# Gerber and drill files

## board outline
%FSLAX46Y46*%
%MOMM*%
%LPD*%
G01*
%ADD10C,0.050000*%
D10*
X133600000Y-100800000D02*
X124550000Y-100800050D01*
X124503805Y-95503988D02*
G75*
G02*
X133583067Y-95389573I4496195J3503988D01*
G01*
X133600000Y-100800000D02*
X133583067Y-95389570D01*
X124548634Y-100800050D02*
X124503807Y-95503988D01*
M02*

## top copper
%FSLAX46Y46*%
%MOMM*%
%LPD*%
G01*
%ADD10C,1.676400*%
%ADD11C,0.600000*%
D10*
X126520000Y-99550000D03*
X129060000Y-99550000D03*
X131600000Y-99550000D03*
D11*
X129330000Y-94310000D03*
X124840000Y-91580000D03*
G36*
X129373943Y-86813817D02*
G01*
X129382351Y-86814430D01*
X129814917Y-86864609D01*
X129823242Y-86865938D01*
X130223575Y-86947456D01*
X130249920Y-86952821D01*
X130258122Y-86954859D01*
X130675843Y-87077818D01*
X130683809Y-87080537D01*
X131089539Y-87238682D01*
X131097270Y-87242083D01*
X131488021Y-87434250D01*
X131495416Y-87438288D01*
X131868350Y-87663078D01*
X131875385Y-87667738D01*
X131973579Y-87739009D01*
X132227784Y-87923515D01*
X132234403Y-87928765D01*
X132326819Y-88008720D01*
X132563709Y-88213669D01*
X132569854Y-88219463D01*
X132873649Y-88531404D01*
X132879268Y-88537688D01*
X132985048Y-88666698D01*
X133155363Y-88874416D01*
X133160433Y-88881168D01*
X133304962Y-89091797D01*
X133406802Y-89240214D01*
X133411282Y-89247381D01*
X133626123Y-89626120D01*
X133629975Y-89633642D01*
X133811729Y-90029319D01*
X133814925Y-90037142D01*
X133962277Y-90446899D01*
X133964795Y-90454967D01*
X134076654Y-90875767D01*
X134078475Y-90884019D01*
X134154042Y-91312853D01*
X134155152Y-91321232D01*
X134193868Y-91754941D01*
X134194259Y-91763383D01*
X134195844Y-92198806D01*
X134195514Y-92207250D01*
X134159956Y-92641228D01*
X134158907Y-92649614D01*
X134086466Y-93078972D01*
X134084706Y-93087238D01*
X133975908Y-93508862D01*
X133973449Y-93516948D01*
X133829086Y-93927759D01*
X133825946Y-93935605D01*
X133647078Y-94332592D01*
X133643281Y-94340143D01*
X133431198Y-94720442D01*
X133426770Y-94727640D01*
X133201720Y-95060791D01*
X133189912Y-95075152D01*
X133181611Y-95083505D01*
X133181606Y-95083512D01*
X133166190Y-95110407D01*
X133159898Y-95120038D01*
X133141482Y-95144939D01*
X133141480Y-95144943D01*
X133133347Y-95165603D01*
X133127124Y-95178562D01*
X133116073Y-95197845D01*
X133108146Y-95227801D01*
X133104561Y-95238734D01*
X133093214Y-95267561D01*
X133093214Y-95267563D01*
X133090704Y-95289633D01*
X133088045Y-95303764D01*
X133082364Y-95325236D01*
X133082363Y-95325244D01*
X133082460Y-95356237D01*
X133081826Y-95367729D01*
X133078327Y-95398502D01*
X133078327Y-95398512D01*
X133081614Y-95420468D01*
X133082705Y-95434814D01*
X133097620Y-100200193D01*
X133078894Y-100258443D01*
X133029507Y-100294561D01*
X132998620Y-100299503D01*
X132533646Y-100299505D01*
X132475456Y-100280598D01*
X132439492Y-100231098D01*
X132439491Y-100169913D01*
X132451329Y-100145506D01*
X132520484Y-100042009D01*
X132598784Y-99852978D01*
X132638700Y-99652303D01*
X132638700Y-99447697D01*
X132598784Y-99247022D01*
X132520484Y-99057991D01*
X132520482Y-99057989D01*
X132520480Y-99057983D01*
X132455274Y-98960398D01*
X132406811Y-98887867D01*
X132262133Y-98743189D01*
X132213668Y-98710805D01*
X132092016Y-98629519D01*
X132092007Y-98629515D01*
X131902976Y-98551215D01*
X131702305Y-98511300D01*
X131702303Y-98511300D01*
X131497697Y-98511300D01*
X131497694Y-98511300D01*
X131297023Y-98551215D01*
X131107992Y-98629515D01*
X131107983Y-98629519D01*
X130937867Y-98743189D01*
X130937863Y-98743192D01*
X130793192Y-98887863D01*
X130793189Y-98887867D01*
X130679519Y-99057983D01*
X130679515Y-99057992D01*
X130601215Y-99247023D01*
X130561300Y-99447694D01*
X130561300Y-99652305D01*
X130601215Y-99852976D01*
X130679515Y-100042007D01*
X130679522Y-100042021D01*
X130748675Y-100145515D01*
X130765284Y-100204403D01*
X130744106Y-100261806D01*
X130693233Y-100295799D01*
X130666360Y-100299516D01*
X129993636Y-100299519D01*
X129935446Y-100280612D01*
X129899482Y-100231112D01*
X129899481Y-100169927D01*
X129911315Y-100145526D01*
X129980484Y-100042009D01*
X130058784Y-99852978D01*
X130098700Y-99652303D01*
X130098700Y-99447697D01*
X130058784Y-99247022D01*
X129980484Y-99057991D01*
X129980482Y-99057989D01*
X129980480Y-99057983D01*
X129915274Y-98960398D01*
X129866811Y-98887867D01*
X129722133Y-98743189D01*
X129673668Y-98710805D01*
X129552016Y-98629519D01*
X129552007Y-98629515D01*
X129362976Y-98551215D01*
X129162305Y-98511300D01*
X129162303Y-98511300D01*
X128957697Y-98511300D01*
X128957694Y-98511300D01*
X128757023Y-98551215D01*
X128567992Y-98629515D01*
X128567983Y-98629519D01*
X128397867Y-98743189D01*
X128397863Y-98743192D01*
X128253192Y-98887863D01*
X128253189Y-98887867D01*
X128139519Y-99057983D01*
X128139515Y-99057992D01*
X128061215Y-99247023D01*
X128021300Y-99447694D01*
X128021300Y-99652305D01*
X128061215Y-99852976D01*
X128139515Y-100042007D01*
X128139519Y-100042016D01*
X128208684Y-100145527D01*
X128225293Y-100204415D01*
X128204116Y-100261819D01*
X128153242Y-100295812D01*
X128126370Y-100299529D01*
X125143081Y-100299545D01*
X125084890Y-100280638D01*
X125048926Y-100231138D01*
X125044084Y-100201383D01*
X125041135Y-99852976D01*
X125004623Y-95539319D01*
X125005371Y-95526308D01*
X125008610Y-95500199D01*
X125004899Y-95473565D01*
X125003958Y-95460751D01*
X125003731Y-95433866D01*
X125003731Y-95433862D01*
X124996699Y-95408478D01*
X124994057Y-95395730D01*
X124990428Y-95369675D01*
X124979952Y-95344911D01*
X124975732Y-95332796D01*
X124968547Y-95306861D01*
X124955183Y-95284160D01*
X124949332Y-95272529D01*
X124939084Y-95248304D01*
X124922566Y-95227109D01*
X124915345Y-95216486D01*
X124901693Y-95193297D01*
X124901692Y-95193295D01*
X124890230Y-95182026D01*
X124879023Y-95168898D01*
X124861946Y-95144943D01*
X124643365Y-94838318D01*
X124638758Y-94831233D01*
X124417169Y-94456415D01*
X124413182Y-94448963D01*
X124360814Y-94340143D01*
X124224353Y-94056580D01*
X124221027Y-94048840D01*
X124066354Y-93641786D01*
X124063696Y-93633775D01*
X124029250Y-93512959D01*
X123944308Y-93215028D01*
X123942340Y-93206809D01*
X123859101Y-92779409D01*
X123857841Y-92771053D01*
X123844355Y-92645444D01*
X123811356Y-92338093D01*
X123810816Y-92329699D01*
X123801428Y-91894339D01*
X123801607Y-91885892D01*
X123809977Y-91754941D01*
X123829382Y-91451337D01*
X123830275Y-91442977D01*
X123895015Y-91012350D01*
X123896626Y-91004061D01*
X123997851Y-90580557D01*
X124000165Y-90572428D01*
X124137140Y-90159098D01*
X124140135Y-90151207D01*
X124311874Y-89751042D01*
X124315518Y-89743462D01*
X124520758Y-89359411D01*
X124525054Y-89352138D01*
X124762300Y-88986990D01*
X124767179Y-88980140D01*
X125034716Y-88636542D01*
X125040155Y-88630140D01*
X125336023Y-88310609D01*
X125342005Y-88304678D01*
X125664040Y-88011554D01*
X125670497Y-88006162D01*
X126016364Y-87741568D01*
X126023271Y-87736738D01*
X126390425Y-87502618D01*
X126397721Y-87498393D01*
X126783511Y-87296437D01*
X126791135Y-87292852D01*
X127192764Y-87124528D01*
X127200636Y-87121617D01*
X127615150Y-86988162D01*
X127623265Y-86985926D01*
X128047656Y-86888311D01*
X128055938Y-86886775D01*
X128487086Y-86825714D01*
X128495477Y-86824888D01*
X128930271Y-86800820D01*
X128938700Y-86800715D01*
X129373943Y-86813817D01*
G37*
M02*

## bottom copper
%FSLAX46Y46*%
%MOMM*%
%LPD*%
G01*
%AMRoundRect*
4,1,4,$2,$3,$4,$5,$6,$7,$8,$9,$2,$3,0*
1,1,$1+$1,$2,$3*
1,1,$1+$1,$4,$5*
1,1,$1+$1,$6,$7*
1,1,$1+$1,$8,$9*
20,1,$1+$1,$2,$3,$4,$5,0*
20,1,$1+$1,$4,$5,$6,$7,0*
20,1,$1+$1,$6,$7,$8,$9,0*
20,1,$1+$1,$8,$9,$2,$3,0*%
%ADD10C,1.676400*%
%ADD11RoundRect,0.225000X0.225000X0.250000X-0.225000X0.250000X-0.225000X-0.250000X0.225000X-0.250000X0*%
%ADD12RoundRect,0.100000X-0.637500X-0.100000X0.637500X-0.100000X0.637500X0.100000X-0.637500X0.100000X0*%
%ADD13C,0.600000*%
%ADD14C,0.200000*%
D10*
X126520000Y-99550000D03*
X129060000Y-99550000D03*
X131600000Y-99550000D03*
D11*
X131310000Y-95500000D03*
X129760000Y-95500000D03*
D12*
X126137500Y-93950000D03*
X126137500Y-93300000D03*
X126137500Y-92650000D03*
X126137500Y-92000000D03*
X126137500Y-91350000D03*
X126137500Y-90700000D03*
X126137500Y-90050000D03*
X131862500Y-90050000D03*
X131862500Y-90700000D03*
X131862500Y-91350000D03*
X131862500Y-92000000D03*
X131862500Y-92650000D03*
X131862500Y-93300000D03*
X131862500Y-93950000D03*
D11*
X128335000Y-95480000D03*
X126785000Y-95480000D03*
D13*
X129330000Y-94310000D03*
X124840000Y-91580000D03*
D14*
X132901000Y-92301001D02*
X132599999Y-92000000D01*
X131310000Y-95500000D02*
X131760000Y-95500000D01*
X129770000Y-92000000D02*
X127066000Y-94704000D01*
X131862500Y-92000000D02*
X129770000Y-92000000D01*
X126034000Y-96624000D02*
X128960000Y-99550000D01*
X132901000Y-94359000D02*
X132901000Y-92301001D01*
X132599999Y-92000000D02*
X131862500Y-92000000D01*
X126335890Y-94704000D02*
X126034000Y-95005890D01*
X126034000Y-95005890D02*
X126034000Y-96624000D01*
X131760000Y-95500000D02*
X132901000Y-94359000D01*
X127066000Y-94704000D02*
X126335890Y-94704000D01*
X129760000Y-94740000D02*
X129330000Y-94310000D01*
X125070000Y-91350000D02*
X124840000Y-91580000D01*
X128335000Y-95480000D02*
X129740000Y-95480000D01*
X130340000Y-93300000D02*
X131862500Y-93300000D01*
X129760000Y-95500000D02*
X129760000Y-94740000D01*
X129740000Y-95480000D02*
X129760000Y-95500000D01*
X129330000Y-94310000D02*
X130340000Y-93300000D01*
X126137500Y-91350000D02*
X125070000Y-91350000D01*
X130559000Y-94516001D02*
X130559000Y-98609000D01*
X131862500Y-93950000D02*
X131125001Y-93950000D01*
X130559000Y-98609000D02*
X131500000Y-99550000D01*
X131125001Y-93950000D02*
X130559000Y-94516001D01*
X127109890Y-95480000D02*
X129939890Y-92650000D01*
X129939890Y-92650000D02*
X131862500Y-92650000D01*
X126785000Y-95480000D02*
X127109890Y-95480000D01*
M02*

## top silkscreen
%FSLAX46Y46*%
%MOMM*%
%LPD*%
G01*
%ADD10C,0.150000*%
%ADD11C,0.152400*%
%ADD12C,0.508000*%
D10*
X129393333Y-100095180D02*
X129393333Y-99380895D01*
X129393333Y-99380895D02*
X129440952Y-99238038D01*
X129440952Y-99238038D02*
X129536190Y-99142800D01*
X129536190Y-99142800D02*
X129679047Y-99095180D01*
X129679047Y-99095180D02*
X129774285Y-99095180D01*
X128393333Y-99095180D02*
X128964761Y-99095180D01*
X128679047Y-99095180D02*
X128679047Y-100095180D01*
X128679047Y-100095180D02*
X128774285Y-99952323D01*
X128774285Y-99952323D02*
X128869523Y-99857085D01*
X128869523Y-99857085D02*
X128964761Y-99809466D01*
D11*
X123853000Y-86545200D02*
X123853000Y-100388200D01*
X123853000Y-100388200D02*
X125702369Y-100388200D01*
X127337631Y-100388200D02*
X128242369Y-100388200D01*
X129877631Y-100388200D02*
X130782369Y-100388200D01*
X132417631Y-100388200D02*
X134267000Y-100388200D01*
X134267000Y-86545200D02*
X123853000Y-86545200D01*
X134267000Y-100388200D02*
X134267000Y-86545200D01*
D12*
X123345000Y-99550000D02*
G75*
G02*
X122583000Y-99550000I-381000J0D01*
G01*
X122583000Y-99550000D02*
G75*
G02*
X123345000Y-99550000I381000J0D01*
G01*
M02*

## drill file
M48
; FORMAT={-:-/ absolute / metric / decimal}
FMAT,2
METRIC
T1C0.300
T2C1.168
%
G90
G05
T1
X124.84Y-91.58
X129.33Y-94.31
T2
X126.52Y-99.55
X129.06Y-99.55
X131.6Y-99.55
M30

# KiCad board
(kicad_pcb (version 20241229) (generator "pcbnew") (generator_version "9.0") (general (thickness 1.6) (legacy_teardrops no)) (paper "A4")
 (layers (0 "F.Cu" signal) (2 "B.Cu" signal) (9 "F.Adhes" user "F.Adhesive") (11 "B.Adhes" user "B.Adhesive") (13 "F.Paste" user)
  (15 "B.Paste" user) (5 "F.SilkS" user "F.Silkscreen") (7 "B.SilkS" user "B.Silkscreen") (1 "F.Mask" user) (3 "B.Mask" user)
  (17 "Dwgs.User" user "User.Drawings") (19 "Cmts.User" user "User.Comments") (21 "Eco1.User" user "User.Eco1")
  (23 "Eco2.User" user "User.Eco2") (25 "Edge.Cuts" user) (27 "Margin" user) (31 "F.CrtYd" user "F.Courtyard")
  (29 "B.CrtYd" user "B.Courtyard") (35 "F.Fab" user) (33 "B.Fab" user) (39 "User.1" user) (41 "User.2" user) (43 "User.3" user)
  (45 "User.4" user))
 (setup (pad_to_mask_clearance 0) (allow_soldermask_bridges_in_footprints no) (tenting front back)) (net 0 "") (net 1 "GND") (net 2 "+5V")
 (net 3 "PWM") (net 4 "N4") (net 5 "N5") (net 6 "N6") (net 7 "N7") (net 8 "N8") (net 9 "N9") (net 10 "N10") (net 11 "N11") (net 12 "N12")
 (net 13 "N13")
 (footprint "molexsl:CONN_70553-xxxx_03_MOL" (layer "F.Cu") (at 126.52 99.55 180)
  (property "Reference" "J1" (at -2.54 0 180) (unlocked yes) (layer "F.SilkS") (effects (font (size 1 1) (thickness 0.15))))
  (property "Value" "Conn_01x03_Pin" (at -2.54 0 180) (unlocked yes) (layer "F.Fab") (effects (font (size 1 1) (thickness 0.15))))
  (fp_line (start 2.667 13.0048) (end 2.667 -0.8382) (stroke (width 0.1524) (type solid)) (layer "F.SilkS"))
  (fp_line (start 2.667 -0.8382) (end 0.817631 -0.8382) (stroke (width 0.1524) (type solid)) (layer "F.SilkS"))
  (fp_line (start -0.817631 -0.8382) (end -1.722369 -0.8382) (stroke (width 0.1524) (type solid)) (layer "F.SilkS"))
  (fp_line (start -3.357631 -0.8382) (end -4.262369 -0.8382) (stroke (width 0.1524) (type solid)) (layer "F.SilkS"))
  (fp_line (start -5.897631 -0.8382) (end -7.747 -0.8382) (stroke (width 0.1524) (type solid)) (layer "F.SilkS"))
  (fp_line (start -7.747 13.0048) (end 2.667 13.0048) (stroke (width 0.1524) (type solid)) (layer "F.SilkS"))
  (fp_line (start -7.747 -0.8382) (end -7.747 13.0048) (stroke (width 0.1524) (type solid)) (layer "F.SilkS"))
  (fp_circle (center 3.556 0) (end 3.937 0) (stroke (width 0.508) (type solid)) (fill no) (layer "F.SilkS"))
  (pad "1" thru_hole circle (at 0 0 180) (size 1.6764 1.6764) (drill 1.1684) (layers "*.Cu" "*.Mask") (remove_unused_layers no)
   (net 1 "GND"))
  (pad "2" thru_hole circle (at -2.54 0 180) (size 1.6764 1.6764) (drill 1.1684) (layers "*.Cu" "*.Mask") (remove_unused_layers no)
   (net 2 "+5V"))
  (pad "3" thru_hole circle (at -5.08 0 180) (size 1.6764 1.6764) (drill 1.1684) (layers "*.Cu" "*.Mask") (remove_unused_layers no)
   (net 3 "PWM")))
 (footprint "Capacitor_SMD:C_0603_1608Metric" (layer "B.Cu") (at 130.535 95.5 180)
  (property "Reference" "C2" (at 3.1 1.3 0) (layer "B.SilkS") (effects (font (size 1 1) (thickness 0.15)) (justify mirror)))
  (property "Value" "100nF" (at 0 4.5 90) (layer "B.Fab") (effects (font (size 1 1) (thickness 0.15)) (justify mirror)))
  (pad "1" smd roundrect (at -0.775 0 180) (size 0.9 0.95) (layers "B.Cu" "B.Mask" "B.Paste") (roundrect_rratio 0.25) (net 2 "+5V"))
  (pad "2" smd roundrect (at 0.775 0 180) (size 0.9 0.95) (layers "B.Cu" "B.Mask" "B.Paste") (roundrect_rratio 0.25) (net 1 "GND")))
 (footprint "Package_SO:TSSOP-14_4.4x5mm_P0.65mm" (layer "B.Cu") (at 129 92)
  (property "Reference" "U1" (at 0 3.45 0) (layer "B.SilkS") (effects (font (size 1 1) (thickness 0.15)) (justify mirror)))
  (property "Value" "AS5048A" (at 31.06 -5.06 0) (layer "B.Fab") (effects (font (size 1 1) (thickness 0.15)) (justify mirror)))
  (pad "1" smd roundrect (at -2.8625 1.95) (size 1.475 0.4) (layers "B.Cu" "B.Mask" "B.Paste") (roundrect_rratio 0.25) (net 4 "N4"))
  (pad "2" smd roundrect (at -2.8625 1.3) (size 1.475 0.4) (layers "B.Cu" "B.Mask" "B.Paste") (roundrect_rratio 0.25) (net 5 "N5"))
  (pad "3" smd roundrect (at -2.8625 0.65) (size 1.475 0.4) (layers "B.Cu" "B.Mask" "B.Paste") (roundrect_rratio 0.25) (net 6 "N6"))
  (pad "4" smd roundrect (at -2.8625 0) (size 1.475 0.4) (layers "B.Cu" "B.Mask" "B.Paste") (roundrect_rratio 0.25) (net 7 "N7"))
  (pad "5" smd roundrect (at -2.8625 -0.65) (size 1.475 0.4) (layers "B.Cu" "B.Mask" "B.Paste") (roundrect_rratio 0.25) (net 1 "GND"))
  (pad "6" smd roundrect (at -2.8625 -1.3) (size 1.475 0.4) (layers "B.Cu" "B.Mask" "B.Paste") (roundrect_rratio 0.25) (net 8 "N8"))
  (pad "7" smd roundrect (at -2.8625 -1.95) (size 1.475 0.4) (layers "B.Cu" "B.Mask" "B.Paste") (roundrect_rratio 0.25) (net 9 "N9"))
  (pad "8" smd roundrect (at 2.8625 -1.95) (size 1.475 0.4) (layers "B.Cu" "B.Mask" "B.Paste") (roundrect_rratio 0.25) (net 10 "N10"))
  (pad "9" smd roundrect (at 2.8625 -1.3) (size 1.475 0.4) (layers "B.Cu" "B.Mask" "B.Paste") (roundrect_rratio 0.25) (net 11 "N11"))
  (pad "10" smd roundrect (at 2.8625 -0.65) (size 1.475 0.4) (layers "B.Cu" "B.Mask" "B.Paste") (roundrect_rratio 0.25) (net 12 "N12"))
  (pad "11" smd roundrect (at 2.8625 0) (size 1.475 0.4) (layers "B.Cu" "B.Mask" "B.Paste") (roundrect_rratio 0.25) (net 2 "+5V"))
  (pad "12" smd roundrect (at 2.8625 0.65) (size 1.475 0.4) (layers "B.Cu" "B.Mask" "B.Paste") (roundrect_rratio 0.25) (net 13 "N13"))
  (pad "13" smd roundrect (at 2.8625 1.3) (size 1.475 0.4) (layers "B.Cu" "B.Mask" "B.Paste") (roundrect_rratio 0.25) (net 1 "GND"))
  (pad "14" smd roundrect (at 2.8625 1.95) (size 1.475 0.4) (layers "B.Cu" "B.Mask" "B.Paste") (roundrect_rratio 0.25) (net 3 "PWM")))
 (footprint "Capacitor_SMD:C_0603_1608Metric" (layer "B.Cu") (at 127.56 95.48 180)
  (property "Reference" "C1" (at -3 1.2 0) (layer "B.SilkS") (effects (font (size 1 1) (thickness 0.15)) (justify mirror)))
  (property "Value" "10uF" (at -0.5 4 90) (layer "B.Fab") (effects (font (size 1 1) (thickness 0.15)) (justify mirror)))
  (pad "1" smd roundrect (at -0.775 0 180) (size 0.9 0.95) (layers "B.Cu" "B.Mask" "B.Paste") (roundrect_rratio 0.25) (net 1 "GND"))
  (pad "2" smd roundrect (at 0.775 0 180) (size 0.9 0.95) (layers "B.Cu" "B.Mask" "B.Paste") (roundrect_rratio 0.25) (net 13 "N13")))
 (gr_line (start 133.6 100.8) (end 124.55 100.80005) (stroke (width 0.05) (type default)) (layer "Edge.Cuts"))
 (gr_arc (start 124.503805 95.503988) (mid 128.928171 86.300128) (end 133.583067 95.389573) (stroke (width 0.05) (type default))
  (layer "Edge.Cuts"))
 (gr_line (start 133.6 100.8) (end 133.583067 95.38957) (stroke (width 0.05) (type default)) (layer "Edge.Cuts"))
 (gr_line (start 124.548634 100.80005) (end 124.503807 95.503988) (stroke (width 0.05) (type default)) (layer "Edge.Cuts"))
 (segment (start 132.901 92.301001) (end 132.599999 92) (width 0.2) (layer "B.Cu") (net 2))
 (segment (start 131.31 95.5) (end 131.76 95.5) (width 0.2) (layer "B.Cu") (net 2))
 (segment (start 129.77 92) (end 127.066 94.704) (width 0.2) (layer "B.Cu") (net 2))
 (segment (start 131.8625 92) (end 129.77 92) (width 0.2) (layer "B.Cu") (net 2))
 (segment (start 126.034 96.624) (end 128.96 99.55) (width 0.2) (layer "B.Cu") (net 2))
 (segment (start 132.901 94.359) (end 132.901 92.301001) (width 0.2) (layer "B.Cu") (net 2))
 (segment (start 132.599999 92) (end 131.8625 92) (width 0.2) (layer "B.Cu") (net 2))
 (segment (start 126.33589 94.704) (end 126.034 95.00589) (width 0.2) (layer "B.Cu") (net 2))
 (segment (start 126.034 95.00589) (end 126.034 96.624) (width 0.2) (layer "B.Cu") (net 2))
 (segment (start 131.76 95.5) (end 132.901 94.359) (width 0.2) (layer "B.Cu") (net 2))
 (segment (start 127.066 94.704) (end 126.33589 94.704) (width 0.2) (layer "B.Cu") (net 2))
 (via (at 129.33 94.31) (size 0.6) (drill 0.3) (layers "F.Cu" "B.Cu") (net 1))
 (via (at 124.84 91.58) (size 0.6) (drill 0.3) (layers "F.Cu" "B.Cu") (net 1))
 (segment (start 129.76 94.74) (end 129.33 94.31) (width 0.2) (layer "B.Cu") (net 1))
 (segment (start 125.07 91.35) (end 124.84 91.58) (width 0.2) (layer "B.Cu") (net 1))
 (segment (start 128.335 95.48) (end 129.74 95.48) (width 0.2) (layer "B.Cu") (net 1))
 (segment (start 130.34 93.3) (end 131.8625 93.3) (width 0.2) (layer "B.Cu") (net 1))
 (segment (start 129.76 95.5) (end 129.76 94.74) (width 0.2) (layer "B.Cu") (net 1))
 (segment (start 129.74 95.48) (end 129.76 95.5) (width 0.2) (layer "B.Cu") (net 1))
 (segment (start 129.33 94.31) (end 130.34 93.3) (width 0.2) (layer "B.Cu") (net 1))
 (segment (start 126.1375 91.35) (end 125.07 91.35) (width 0.2) (layer "B.Cu") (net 1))
 (segment (start 130.559 94.516001) (end 130.559 98.609) (width 0.2) (layer "B.Cu") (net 3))
 (segment (start 131.8625 93.95) (end 131.125001 93.95) (width 0.2) (layer "B.Cu") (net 3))
 (segment (start 130.559 98.609) (end 131.5 99.55) (width 0.2) (layer "B.Cu") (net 3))
 (segment (start 131.125001 93.95) (end 130.559 94.516001) (width 0.2) (layer "B.Cu") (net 3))
 (segment (start 127.10989 95.48) (end 129.93989 92.65) (width 0.2) (layer "B.Cu") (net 13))
 (segment (start 129.93989 92.65) (end 131.8625 92.65) (width 0.2) (layer "B.Cu") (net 13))
 (segment (start 126.785 95.48) (end 127.10989 95.48) (width 0.2) (layer "B.Cu") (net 13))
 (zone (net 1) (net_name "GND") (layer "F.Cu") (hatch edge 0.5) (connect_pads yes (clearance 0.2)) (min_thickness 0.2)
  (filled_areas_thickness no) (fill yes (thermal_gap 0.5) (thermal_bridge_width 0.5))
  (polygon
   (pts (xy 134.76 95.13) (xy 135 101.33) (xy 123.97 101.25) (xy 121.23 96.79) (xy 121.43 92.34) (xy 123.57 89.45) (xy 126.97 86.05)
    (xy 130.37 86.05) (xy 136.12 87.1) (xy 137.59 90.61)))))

